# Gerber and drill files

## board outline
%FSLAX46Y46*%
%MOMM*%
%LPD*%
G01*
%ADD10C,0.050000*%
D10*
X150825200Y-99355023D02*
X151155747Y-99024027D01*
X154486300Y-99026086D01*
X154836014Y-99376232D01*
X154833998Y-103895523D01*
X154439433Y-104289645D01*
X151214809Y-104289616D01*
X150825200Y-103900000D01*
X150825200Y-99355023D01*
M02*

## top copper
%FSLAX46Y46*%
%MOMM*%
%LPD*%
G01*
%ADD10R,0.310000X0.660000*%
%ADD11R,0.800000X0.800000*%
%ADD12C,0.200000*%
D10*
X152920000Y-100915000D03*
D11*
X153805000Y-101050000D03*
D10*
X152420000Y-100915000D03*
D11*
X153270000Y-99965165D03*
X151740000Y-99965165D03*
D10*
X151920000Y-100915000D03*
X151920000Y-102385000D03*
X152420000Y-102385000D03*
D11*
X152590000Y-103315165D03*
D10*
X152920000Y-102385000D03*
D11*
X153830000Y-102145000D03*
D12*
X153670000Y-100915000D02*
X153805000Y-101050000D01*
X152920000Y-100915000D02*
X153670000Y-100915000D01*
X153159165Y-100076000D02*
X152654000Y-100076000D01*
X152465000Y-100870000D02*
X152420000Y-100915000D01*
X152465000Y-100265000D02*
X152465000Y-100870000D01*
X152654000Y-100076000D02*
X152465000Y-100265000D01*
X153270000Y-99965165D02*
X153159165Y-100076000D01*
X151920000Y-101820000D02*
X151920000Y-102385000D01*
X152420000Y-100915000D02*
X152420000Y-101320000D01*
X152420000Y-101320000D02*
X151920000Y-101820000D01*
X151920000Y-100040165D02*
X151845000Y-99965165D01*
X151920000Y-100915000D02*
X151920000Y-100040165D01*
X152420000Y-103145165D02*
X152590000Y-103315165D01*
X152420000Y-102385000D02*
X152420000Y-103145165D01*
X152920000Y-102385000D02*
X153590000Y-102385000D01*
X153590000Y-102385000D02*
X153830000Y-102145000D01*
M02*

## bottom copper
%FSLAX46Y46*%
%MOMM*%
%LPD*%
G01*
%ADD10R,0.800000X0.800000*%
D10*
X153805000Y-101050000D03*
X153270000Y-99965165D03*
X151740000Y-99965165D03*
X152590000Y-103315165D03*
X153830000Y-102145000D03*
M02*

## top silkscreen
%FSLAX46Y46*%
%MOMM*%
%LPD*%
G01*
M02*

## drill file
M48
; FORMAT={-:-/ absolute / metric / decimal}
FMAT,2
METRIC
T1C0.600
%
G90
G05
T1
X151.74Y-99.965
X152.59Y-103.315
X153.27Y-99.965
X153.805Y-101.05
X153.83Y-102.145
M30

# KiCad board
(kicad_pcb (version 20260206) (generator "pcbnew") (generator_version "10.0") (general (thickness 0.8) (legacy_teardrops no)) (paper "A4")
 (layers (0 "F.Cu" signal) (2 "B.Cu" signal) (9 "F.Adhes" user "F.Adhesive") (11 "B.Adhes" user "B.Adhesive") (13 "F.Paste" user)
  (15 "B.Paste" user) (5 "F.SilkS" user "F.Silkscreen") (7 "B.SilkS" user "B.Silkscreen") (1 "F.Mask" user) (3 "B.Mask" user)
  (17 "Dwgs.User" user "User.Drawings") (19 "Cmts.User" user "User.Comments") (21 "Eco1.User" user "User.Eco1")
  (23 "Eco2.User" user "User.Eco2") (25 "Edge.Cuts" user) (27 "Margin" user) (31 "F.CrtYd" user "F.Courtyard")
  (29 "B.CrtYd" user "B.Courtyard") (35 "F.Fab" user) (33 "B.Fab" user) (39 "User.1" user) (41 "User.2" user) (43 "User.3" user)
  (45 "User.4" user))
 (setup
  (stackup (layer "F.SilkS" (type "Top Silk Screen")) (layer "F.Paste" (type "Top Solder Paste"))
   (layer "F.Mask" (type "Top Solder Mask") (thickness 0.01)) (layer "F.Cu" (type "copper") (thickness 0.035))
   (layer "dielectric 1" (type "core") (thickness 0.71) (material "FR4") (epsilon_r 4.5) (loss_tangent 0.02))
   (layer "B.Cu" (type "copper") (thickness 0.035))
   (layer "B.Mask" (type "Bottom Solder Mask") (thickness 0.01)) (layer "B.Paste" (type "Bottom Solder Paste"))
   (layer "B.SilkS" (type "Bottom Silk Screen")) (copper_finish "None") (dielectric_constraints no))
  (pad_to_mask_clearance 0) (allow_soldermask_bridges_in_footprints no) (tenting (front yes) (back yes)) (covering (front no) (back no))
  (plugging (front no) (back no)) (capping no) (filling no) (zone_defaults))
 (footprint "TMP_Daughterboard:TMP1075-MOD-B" (layer "F.Cu") (at 152.4 101.6)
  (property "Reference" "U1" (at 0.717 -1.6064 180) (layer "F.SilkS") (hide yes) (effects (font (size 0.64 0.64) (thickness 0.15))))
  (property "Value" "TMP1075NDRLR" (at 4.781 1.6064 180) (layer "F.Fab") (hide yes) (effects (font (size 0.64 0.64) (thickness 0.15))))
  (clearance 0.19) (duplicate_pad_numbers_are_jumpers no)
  (pad "1" smd rect (at 0.52 -0.685 270) (size 0.66 0.31) (layers "F.Cu" "F.Mask" "F.Paste") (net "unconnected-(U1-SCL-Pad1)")
   (solder_mask_margin 0.08))
  (pad "1" thru_hole rect (at 1.405 -0.55 180) (size 0.8 0.8) (drill 0.6) (layers "*.Cu" "*.Mask") (remove_unused_layers no)
   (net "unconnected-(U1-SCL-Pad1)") (solder_mask_margin 0.102))
  (pad "2" smd rect (at 0.02 -0.685 270) (size 0.66 0.31) (layers "F.Cu" "F.Mask" "F.Paste") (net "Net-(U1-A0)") (solder_mask_margin 0.08))
  (pad "2" thru_hole rect (at 0.87 -1.634835) (size 0.8 0.8) (drill 0.6) (layers "*.Cu" "*.Mask") (remove_unused_layers no)
   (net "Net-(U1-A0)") (solder_mask_margin 0.102))
  (pad "3" thru_hole rect (at -0.66 -1.634835 90) (size 0.8 0.8) (drill 0.6) (layers "*.Cu" "*.Mask") (remove_unused_layers no)
   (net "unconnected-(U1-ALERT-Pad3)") (solder_mask_margin 0.102))
  (pad "3" smd rect (at -0.48 -0.685 270) (size 0.66 0.31) (layers "F.Cu" "F.Mask" "F.Paste") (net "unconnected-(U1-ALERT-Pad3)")
   (solder_mask_margin 0.08))
  (pad "4" smd rect (at -0.48 0.785 270) (size 0.66 0.31) (layers "F.Cu" "F.Mask" "F.Paste") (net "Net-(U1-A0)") (solder_mask_margin 0.08))
  (pad "5" smd rect (at 0.02 0.785 90) (size 0.66 0.31) (layers "F.Cu" "F.Mask" "F.Paste") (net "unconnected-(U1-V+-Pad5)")
   (solder_mask_margin 0.08))
  (pad "5" thru_hole rect (at 0.19 1.715165 270) (size 0.8 0.8) (drill 0.6) (layers "*.Cu" "*.Mask") (remove_unused_layers no)
   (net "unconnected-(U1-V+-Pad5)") (solder_mask_margin 0.102))
  (pad "6" smd rect (at 0.52 0.785 270) (size 0.66 0.31) (layers "F.Cu" "F.Mask" "F.Paste") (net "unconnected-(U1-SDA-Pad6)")
   (solder_mask_margin 0.08))
  (pad "6" thru_hole rect (at 1.43 0.545 180) (size 0.8 0.8) (drill 0.6) (layers "*.Cu" "*.Mask") (remove_unused_layers no)
   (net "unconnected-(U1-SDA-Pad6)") (solder_mask_margin 0.102)))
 (gr_poly
  (pts (xy 150.8252 99.355023) (xy 151.155747 99.024027) (xy 154.4863 99.026086) (xy 154.836014 99.376232) (xy 154.833998 103.895523)
   (xy 154.439433 104.289645) (xy 151.214809 104.289616) (xy 150.8252 103.9))
  (stroke (width 0.05) (type solid)) (fill no) (layer "Edge.Cuts"))
 (segment (start 153.67 100.915) (end 153.805 101.05) (width 0.2) (layer "F.Cu") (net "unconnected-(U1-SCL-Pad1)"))
 (segment (start 152.92 100.915) (end 153.67 100.915) (width 0.2) (layer "F.Cu") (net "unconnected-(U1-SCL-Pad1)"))
 (segment (start 153.159165 100.076) (end 152.654 100.076) (width 0.2) (layer "F.Cu") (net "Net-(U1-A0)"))
 (segment (start 152.465 100.87) (end 152.42 100.915) (width 0.2) (layer "F.Cu") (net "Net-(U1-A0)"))
 (segment (start 152.465 100.265) (end 152.465 100.87) (width 0.2) (layer "F.Cu") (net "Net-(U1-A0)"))
 (segment (start 152.654 100.076) (end 152.465 100.265) (width 0.2) (layer "F.Cu") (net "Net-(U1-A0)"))
 (segment (start 153.27 99.965165) (end 153.159165 100.076) (width 0.2) (layer "F.Cu") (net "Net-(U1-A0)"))
 (segment (start 151.92 101.82) (end 151.92 102.385) (width 0.2) (layer "F.Cu") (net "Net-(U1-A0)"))
 (segment (start 152.42 100.915) (end 152.42 101.32) (width 0.2) (layer "F.Cu") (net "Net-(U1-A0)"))
 (segment (start 152.42 101.32) (end 151.92 101.82) (width 0.2) (layer "F.Cu") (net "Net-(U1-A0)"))
 (segment (start 151.92 100.040165) (end 151.845 99.965165) (width 0.2) (layer "F.Cu") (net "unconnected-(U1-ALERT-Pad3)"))
 (segment (start 151.92 100.915) (end 151.92 100.040165) (width 0.2) (layer "F.Cu") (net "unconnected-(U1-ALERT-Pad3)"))
 (segment (start 152.42 103.145165) (end 152.59 103.315165) (width 0.2) (layer "F.Cu") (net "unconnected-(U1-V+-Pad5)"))
 (segment (start 152.42 102.385) (end 152.42 103.145165) (width 0.2) (layer "F.Cu") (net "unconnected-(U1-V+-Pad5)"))
 (segment (start 152.92 102.385) (end 153.59 102.385) (width 0.2) (layer "F.Cu") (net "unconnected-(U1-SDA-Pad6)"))
 (segment (start 153.59 102.385) (end 153.83 102.145) (width 0.2) (layer "F.Cu") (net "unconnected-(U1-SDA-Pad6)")))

